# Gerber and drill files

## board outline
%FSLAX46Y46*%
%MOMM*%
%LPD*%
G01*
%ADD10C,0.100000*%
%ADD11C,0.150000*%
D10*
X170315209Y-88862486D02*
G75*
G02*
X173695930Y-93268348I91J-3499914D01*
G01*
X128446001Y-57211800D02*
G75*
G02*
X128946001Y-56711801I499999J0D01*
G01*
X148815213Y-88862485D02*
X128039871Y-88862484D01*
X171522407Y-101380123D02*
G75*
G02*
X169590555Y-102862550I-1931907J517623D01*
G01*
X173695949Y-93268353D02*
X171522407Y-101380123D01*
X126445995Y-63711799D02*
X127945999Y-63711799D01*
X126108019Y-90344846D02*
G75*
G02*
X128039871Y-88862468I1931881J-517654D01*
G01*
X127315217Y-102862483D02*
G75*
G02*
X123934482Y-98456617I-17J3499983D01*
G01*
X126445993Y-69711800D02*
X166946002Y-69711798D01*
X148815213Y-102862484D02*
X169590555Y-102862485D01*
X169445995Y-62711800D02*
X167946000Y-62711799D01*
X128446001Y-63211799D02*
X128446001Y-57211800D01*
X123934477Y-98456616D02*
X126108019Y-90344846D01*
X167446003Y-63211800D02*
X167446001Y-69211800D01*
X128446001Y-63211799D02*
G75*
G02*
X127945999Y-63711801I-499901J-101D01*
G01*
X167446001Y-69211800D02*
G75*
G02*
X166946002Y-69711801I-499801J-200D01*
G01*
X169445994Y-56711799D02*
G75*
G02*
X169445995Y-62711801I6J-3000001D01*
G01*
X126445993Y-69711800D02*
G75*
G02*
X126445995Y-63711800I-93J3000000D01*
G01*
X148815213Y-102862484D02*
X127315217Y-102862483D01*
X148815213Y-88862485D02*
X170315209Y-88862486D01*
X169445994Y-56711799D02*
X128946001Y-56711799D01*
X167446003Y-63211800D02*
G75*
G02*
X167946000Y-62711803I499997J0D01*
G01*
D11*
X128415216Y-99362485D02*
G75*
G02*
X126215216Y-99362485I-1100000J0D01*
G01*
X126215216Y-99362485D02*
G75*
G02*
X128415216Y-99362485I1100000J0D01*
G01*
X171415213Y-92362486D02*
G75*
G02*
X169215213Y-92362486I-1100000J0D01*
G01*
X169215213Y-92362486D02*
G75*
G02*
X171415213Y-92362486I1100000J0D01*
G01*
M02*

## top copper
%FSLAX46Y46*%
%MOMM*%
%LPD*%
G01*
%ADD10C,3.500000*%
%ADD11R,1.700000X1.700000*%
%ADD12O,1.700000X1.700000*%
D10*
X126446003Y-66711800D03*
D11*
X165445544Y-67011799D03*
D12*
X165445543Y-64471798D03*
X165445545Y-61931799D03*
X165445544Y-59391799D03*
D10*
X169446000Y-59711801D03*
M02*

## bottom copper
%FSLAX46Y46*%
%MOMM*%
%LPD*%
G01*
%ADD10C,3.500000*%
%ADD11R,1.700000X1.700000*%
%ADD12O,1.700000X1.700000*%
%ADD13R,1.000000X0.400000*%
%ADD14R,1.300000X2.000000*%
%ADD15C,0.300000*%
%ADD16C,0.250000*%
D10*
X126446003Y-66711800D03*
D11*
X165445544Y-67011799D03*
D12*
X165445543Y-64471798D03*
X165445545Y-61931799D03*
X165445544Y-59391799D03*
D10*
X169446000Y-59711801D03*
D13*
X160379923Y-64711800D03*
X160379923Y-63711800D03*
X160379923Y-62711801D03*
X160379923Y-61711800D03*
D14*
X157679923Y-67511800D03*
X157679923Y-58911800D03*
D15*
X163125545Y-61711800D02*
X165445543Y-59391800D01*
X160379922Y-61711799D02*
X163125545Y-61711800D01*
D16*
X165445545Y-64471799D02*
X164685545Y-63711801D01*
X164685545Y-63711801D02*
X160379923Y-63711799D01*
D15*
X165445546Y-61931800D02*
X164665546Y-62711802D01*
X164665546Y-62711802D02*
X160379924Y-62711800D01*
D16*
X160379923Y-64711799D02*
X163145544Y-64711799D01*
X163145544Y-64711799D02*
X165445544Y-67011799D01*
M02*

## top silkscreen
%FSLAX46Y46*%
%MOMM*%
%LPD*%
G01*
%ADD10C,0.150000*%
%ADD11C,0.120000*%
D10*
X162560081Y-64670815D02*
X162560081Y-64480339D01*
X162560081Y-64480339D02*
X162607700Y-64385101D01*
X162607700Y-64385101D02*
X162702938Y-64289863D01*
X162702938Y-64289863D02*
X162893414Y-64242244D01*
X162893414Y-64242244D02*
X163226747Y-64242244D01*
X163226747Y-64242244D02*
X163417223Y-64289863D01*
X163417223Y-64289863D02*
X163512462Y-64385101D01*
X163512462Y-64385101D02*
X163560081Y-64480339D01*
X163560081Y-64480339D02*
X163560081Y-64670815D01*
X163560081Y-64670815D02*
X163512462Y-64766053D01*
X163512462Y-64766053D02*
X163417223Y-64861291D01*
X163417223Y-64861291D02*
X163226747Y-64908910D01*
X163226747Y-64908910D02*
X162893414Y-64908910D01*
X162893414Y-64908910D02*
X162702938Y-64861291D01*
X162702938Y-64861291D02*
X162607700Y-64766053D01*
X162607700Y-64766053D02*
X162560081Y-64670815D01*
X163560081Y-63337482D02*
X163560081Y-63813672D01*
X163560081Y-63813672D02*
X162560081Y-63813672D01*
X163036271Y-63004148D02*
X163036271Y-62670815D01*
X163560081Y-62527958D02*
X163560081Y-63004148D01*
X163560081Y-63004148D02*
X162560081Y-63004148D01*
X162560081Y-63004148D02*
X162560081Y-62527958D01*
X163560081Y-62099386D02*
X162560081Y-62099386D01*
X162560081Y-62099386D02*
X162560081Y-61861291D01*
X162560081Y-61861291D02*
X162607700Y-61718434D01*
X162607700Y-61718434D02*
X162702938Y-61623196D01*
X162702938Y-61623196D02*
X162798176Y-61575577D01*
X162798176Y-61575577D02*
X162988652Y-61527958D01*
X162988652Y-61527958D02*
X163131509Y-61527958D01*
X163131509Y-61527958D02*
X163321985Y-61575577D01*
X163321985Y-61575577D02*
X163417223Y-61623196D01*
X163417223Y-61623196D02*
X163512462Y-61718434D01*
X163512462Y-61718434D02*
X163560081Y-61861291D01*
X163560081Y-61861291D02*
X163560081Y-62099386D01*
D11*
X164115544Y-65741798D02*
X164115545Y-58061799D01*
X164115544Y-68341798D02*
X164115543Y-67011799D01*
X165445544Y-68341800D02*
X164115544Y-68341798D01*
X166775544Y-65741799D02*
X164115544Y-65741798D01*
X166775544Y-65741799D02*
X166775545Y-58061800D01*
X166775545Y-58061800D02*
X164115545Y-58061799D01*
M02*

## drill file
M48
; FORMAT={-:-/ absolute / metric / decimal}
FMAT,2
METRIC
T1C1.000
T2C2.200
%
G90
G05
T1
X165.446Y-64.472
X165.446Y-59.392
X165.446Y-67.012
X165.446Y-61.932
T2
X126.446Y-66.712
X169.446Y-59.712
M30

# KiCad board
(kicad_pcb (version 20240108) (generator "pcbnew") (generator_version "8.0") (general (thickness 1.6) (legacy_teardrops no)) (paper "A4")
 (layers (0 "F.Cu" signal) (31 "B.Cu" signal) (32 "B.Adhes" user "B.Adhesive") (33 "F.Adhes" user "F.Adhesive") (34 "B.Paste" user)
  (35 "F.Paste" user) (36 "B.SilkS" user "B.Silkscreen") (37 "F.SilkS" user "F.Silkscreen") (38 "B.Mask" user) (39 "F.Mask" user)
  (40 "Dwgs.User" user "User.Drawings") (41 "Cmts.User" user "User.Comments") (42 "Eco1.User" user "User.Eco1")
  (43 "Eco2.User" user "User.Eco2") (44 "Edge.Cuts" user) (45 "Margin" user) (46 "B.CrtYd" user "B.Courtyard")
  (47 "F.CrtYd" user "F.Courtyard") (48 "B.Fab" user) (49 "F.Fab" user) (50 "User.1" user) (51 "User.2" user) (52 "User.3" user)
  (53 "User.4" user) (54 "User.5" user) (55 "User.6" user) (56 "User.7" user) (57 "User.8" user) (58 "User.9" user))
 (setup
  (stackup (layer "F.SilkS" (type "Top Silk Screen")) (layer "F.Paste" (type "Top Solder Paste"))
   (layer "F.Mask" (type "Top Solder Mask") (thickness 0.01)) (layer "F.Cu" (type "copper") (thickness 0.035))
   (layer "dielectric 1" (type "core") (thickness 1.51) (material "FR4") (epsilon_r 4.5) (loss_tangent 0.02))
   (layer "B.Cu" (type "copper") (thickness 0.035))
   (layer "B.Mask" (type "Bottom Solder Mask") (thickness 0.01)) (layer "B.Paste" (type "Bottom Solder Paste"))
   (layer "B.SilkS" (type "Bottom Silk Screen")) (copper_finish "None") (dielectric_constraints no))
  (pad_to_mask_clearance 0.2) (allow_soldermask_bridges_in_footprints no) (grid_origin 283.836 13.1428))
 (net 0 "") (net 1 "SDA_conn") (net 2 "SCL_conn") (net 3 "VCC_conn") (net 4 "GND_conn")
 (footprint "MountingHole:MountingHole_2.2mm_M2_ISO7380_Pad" (layer "F.Cu") (at 126.446003 66.7118 90)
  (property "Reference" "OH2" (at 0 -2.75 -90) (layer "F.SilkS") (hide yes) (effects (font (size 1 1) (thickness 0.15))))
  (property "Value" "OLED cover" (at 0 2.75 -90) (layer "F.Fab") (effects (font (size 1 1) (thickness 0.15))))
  (pad "1" thru_hole circle (at 0 0 90) (size 3.5 3.5) (drill 2.2) (layers "*.Cu" "*.Mask") (remove_unused_layers no)))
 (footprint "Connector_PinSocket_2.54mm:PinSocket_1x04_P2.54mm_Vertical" (layer "F.Cu") (at 165.445544 67.011799 180)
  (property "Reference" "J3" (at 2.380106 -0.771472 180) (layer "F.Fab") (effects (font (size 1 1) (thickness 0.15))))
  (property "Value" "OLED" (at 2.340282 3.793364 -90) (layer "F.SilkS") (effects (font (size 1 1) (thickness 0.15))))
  (fp_line (start 1.33 1.270001) (end 1.329999 8.95) (stroke (width 0.12) (type solid)) (layer "F.SilkS"))
  (fp_line (start 1.33 -1.329999) (end 1.330001 0) (stroke (width 0.12) (type solid)) (layer "F.SilkS"))
  (fp_line (start 0 -1.330001) (end 1.33 -1.329999) (stroke (width 0.12) (type solid)) (layer "F.SilkS"))
  (fp_line (start -1.33 1.27) (end 1.33 1.270001) (stroke (width 0.12) (type solid)) (layer "F.SilkS"))
  (fp_line (start -1.33 1.27) (end -1.330001 8.949999) (stroke (width 0.12) (type solid)) (layer "F.SilkS"))
  (fp_line (start -1.330001 8.949999) (end 1.329999 8.95) (stroke (width 0.12) (type solid)) (layer "F.SilkS"))
  (pad "1" thru_hole rect (at 0 0 180) (size 1.7 1.7) (drill 1) (layers "*.Cu" "*.Mask") (remove_unused_layers no) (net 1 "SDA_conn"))
  (pad "2" thru_hole oval (at 0.000001 2.540001 180) (size 1.7 1.7) (drill 1) (layers "*.Cu" "*.Mask") (remove_unused_layers no)
   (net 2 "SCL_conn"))
  (pad "3" thru_hole oval (at -0.000001 5.08 180) (size 1.7 1.7) (drill 1) (layers "*.Cu" "*.Mask") (remove_unused_layers no)
   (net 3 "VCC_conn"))
  (pad "4" thru_hole oval (at 0 7.62 180) (size 1.7 1.7) (drill 1) (layers "*.Cu" "*.Mask") (remove_unused_layers no) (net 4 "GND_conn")))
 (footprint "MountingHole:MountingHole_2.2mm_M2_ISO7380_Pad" (layer "F.Cu") (at 169.446 59.711801 90)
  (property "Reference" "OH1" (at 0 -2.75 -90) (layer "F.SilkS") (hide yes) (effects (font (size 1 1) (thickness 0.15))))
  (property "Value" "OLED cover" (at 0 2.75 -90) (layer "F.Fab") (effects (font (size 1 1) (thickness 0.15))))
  (pad "1" thru_hole circle (at 0 0 90) (size 3.5 3.5) (drill 2.2) (layers "*.Cu" "*.Mask") (remove_unused_layers no)))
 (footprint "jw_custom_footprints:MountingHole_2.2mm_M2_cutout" (layer "F.Cu") (at 127.315216 99.362485 180)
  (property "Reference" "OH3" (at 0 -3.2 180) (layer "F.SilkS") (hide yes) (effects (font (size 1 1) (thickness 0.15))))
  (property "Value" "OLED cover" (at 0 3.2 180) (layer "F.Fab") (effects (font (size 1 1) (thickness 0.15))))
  (fp_circle (center 0 0) (end 1.1 0) (stroke (width 0.15) (type solid)) (fill none) (layer "Edge.Cuts")))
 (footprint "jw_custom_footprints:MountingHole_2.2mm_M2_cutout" (layer "F.Cu") (at 170.315213 92.362486)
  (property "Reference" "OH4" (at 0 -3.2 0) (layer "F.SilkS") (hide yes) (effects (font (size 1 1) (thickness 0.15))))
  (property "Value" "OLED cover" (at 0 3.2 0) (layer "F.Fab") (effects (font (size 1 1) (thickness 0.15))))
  (fp_circle (center 0 0) (end 1.1 0) (stroke (width 0.15) (type solid)) (fill none) (layer "Edge.Cuts")))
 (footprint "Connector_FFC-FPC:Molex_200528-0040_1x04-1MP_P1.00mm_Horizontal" (layer "B.Cu") (at 159.469923 63.2118 90)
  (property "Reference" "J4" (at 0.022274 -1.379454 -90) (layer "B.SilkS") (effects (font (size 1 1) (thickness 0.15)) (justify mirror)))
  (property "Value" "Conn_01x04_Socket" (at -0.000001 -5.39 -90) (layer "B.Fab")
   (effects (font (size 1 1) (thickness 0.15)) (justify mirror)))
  (pad "1" smd rect (at -1.5 0.91 90) (size 0.4 1) (layers "B.Cu" "B.Paste" "B.Mask") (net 1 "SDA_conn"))
  (pad "2" smd rect (at -0.5 0.91 90) (size 0.4 1) (layers "B.Cu" "B.Paste" "B.Mask") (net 2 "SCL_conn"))
  (pad "3" smd rect (at 0.499999 0.91 90) (size 0.4 1) (layers "B.Cu" "B.Paste" "B.Mask") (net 3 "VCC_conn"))
  (pad "4" smd rect (at 1.5 0.91 90) (size 0.4 1) (layers "B.Cu" "B.Paste" "B.Mask") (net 4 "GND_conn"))
  (pad "MP" smd rect (at -4.3 -1.79 90) (size 2 1.3) (layers "B.Cu" "B.Paste" "B.Mask"))
  (pad "MP" smd rect (at 4.3 -1.79 90) (size 2 1.3) (layers "B.Cu" "B.Paste" "B.Mask")))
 (gr_arc (start 170.315209 88.862486) (mid 173.092 90.2318) (end 173.695949 93.268353) (stroke (width 0.1) (type default))
  (layer "Edge.Cuts"))
 (gr_arc (start 128.446001 57.2118) (mid 128.592448 56.858236) (end 128.946001 56.711799) (stroke (width 0.1) (type default))
  (layer "Edge.Cuts"))
 (gr_line (start 148.815213 88.862485) (end 128.039871 88.862484) (stroke (width 0.1) (type default)) (layer "Edge.Cuts"))
 (gr_arc (start 171.522407 101.380123) (mid 170.808076 102.449182) (end 169.590555 102.862485) (stroke (width 0.1) (type default))
  (layer "Edge.Cuts"))
 (gr_line (start 173.695949 93.268353) (end 171.522407 101.380123) (stroke (width 0.1) (type solid)) (layer "Edge.Cuts"))
 (gr_line (start 126.445995 63.711799) (end 127.945999 63.711799) (stroke (width 0.1) (type default)) (layer "Edge.Cuts"))
 (gr_arc (start 126.108019 90.344846) (mid 126.822347 89.275774) (end 128.039871 88.862484) (stroke (width 0.1) (type default))
  (layer "Edge.Cuts"))
 (gr_arc (start 127.315217 102.862483) (mid 124.538452 101.493159) (end 123.934477 98.456616) (stroke (width 0.1) (type default))
  (layer "Edge.Cuts"))
 (gr_line (start 126.445993 69.7118) (end 166.946002 69.711798) (stroke (width 0.1) (type default)) (layer "Edge.Cuts"))
 (gr_line (start 148.815213 102.862484) (end 169.590555 102.862485) (stroke (width 0.1) (type default)) (layer "Edge.Cuts"))
 (gr_line (start 169.445995 62.7118) (end 167.946 62.711799) (stroke (width 0.1) (type default)) (layer "Edge.Cuts"))
 (gr_line (start 128.446001 63.211799) (end 128.446001 57.2118) (stroke (width 0.1) (type default)) (layer "Edge.Cuts"))
 (gr_line (start 123.934477 98.456616) (end 126.108019 90.344846) (stroke (width 0.1) (type solid)) (layer "Edge.Cuts"))
 (gr_line (start 167.446003 63.2118) (end 167.446001 69.2118) (stroke (width 0.1) (type default)) (layer "Edge.Cuts"))
 (gr_arc (start 128.446001 63.211799) (mid 128.299561 63.565378) (end 127.945999 63.711799) (stroke (width 0.1) (type default))
  (layer "Edge.Cuts"))
 (gr_arc (start 167.446001 69.2118) (mid 167.299598 69.565408) (end 166.946002 69.711798) (stroke (width 0.1) (type default))
  (layer "Edge.Cuts"))
 (gr_arc (start 169.445994 56.711799) (mid 172.44604 59.71185) (end 169.445995 62.7118) (stroke (width 0.1) (type default))
  (layer "Edge.Cuts"))
 (gr_arc (start 126.445993 69.7118) (mid 123.445889 66.711819) (end 126.445995 63.711799) (stroke (width 0.1) (type default))
  (layer "Edge.Cuts"))
 (gr_line (start 148.815213 102.862484) (end 127.315217 102.862483) (stroke (width 0.1) (type default)) (layer "Edge.Cuts"))
 (gr_line (start 148.815213 88.862485) (end 170.315209 88.862486) (stroke (width 0.1) (type default)) (layer "Edge.Cuts"))
 (gr_line (start 169.445994 56.711799) (end 128.946001 56.711799) (stroke (width 0.1) (type default)) (layer "Edge.Cuts"))
 (gr_arc (start 167.446003 63.2118) (mid 167.592444 62.858233) (end 167.946 62.711799) (stroke (width 0.1) (type default))
  (layer "Edge.Cuts"))
 (segment (start 163.125545 61.7118) (end 165.445543 59.3918) (width 0.3) (layer "B.Cu") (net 4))
 (segment (start 160.379922 61.711799) (end 163.125545 61.7118) (width 0.3) (layer "B.Cu") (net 4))
 (segment (start 165.445545 64.471799) (end 164.685545 63.711801) (width 0.25) (layer "B.Cu") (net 2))
 (segment (start 164.685545 63.711801) (end 160.379923 63.711799) (width 0.25) (layer "B.Cu") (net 2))
 (segment (start 165.445546 61.9318) (end 164.665546 62.711802) (width 0.3) (layer "B.Cu") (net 3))
 (segment (start 164.665546 62.711802) (end 160.379924 62.7118) (width 0.3) (layer "B.Cu") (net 3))
 (segment (start 160.379923 64.711799) (end 163.145544 64.711799) (width 0.25) (layer "B.Cu") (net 1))
 (segment (start 163.145544 64.711799) (end 165.445544 67.011799) (width 0.25) (layer "B.Cu") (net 1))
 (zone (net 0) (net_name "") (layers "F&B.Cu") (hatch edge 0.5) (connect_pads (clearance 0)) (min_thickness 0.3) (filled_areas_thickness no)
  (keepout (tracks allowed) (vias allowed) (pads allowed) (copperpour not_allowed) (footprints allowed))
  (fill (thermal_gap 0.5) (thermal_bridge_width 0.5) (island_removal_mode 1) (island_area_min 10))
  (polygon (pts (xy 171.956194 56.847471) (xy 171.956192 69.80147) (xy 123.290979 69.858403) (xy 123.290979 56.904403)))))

